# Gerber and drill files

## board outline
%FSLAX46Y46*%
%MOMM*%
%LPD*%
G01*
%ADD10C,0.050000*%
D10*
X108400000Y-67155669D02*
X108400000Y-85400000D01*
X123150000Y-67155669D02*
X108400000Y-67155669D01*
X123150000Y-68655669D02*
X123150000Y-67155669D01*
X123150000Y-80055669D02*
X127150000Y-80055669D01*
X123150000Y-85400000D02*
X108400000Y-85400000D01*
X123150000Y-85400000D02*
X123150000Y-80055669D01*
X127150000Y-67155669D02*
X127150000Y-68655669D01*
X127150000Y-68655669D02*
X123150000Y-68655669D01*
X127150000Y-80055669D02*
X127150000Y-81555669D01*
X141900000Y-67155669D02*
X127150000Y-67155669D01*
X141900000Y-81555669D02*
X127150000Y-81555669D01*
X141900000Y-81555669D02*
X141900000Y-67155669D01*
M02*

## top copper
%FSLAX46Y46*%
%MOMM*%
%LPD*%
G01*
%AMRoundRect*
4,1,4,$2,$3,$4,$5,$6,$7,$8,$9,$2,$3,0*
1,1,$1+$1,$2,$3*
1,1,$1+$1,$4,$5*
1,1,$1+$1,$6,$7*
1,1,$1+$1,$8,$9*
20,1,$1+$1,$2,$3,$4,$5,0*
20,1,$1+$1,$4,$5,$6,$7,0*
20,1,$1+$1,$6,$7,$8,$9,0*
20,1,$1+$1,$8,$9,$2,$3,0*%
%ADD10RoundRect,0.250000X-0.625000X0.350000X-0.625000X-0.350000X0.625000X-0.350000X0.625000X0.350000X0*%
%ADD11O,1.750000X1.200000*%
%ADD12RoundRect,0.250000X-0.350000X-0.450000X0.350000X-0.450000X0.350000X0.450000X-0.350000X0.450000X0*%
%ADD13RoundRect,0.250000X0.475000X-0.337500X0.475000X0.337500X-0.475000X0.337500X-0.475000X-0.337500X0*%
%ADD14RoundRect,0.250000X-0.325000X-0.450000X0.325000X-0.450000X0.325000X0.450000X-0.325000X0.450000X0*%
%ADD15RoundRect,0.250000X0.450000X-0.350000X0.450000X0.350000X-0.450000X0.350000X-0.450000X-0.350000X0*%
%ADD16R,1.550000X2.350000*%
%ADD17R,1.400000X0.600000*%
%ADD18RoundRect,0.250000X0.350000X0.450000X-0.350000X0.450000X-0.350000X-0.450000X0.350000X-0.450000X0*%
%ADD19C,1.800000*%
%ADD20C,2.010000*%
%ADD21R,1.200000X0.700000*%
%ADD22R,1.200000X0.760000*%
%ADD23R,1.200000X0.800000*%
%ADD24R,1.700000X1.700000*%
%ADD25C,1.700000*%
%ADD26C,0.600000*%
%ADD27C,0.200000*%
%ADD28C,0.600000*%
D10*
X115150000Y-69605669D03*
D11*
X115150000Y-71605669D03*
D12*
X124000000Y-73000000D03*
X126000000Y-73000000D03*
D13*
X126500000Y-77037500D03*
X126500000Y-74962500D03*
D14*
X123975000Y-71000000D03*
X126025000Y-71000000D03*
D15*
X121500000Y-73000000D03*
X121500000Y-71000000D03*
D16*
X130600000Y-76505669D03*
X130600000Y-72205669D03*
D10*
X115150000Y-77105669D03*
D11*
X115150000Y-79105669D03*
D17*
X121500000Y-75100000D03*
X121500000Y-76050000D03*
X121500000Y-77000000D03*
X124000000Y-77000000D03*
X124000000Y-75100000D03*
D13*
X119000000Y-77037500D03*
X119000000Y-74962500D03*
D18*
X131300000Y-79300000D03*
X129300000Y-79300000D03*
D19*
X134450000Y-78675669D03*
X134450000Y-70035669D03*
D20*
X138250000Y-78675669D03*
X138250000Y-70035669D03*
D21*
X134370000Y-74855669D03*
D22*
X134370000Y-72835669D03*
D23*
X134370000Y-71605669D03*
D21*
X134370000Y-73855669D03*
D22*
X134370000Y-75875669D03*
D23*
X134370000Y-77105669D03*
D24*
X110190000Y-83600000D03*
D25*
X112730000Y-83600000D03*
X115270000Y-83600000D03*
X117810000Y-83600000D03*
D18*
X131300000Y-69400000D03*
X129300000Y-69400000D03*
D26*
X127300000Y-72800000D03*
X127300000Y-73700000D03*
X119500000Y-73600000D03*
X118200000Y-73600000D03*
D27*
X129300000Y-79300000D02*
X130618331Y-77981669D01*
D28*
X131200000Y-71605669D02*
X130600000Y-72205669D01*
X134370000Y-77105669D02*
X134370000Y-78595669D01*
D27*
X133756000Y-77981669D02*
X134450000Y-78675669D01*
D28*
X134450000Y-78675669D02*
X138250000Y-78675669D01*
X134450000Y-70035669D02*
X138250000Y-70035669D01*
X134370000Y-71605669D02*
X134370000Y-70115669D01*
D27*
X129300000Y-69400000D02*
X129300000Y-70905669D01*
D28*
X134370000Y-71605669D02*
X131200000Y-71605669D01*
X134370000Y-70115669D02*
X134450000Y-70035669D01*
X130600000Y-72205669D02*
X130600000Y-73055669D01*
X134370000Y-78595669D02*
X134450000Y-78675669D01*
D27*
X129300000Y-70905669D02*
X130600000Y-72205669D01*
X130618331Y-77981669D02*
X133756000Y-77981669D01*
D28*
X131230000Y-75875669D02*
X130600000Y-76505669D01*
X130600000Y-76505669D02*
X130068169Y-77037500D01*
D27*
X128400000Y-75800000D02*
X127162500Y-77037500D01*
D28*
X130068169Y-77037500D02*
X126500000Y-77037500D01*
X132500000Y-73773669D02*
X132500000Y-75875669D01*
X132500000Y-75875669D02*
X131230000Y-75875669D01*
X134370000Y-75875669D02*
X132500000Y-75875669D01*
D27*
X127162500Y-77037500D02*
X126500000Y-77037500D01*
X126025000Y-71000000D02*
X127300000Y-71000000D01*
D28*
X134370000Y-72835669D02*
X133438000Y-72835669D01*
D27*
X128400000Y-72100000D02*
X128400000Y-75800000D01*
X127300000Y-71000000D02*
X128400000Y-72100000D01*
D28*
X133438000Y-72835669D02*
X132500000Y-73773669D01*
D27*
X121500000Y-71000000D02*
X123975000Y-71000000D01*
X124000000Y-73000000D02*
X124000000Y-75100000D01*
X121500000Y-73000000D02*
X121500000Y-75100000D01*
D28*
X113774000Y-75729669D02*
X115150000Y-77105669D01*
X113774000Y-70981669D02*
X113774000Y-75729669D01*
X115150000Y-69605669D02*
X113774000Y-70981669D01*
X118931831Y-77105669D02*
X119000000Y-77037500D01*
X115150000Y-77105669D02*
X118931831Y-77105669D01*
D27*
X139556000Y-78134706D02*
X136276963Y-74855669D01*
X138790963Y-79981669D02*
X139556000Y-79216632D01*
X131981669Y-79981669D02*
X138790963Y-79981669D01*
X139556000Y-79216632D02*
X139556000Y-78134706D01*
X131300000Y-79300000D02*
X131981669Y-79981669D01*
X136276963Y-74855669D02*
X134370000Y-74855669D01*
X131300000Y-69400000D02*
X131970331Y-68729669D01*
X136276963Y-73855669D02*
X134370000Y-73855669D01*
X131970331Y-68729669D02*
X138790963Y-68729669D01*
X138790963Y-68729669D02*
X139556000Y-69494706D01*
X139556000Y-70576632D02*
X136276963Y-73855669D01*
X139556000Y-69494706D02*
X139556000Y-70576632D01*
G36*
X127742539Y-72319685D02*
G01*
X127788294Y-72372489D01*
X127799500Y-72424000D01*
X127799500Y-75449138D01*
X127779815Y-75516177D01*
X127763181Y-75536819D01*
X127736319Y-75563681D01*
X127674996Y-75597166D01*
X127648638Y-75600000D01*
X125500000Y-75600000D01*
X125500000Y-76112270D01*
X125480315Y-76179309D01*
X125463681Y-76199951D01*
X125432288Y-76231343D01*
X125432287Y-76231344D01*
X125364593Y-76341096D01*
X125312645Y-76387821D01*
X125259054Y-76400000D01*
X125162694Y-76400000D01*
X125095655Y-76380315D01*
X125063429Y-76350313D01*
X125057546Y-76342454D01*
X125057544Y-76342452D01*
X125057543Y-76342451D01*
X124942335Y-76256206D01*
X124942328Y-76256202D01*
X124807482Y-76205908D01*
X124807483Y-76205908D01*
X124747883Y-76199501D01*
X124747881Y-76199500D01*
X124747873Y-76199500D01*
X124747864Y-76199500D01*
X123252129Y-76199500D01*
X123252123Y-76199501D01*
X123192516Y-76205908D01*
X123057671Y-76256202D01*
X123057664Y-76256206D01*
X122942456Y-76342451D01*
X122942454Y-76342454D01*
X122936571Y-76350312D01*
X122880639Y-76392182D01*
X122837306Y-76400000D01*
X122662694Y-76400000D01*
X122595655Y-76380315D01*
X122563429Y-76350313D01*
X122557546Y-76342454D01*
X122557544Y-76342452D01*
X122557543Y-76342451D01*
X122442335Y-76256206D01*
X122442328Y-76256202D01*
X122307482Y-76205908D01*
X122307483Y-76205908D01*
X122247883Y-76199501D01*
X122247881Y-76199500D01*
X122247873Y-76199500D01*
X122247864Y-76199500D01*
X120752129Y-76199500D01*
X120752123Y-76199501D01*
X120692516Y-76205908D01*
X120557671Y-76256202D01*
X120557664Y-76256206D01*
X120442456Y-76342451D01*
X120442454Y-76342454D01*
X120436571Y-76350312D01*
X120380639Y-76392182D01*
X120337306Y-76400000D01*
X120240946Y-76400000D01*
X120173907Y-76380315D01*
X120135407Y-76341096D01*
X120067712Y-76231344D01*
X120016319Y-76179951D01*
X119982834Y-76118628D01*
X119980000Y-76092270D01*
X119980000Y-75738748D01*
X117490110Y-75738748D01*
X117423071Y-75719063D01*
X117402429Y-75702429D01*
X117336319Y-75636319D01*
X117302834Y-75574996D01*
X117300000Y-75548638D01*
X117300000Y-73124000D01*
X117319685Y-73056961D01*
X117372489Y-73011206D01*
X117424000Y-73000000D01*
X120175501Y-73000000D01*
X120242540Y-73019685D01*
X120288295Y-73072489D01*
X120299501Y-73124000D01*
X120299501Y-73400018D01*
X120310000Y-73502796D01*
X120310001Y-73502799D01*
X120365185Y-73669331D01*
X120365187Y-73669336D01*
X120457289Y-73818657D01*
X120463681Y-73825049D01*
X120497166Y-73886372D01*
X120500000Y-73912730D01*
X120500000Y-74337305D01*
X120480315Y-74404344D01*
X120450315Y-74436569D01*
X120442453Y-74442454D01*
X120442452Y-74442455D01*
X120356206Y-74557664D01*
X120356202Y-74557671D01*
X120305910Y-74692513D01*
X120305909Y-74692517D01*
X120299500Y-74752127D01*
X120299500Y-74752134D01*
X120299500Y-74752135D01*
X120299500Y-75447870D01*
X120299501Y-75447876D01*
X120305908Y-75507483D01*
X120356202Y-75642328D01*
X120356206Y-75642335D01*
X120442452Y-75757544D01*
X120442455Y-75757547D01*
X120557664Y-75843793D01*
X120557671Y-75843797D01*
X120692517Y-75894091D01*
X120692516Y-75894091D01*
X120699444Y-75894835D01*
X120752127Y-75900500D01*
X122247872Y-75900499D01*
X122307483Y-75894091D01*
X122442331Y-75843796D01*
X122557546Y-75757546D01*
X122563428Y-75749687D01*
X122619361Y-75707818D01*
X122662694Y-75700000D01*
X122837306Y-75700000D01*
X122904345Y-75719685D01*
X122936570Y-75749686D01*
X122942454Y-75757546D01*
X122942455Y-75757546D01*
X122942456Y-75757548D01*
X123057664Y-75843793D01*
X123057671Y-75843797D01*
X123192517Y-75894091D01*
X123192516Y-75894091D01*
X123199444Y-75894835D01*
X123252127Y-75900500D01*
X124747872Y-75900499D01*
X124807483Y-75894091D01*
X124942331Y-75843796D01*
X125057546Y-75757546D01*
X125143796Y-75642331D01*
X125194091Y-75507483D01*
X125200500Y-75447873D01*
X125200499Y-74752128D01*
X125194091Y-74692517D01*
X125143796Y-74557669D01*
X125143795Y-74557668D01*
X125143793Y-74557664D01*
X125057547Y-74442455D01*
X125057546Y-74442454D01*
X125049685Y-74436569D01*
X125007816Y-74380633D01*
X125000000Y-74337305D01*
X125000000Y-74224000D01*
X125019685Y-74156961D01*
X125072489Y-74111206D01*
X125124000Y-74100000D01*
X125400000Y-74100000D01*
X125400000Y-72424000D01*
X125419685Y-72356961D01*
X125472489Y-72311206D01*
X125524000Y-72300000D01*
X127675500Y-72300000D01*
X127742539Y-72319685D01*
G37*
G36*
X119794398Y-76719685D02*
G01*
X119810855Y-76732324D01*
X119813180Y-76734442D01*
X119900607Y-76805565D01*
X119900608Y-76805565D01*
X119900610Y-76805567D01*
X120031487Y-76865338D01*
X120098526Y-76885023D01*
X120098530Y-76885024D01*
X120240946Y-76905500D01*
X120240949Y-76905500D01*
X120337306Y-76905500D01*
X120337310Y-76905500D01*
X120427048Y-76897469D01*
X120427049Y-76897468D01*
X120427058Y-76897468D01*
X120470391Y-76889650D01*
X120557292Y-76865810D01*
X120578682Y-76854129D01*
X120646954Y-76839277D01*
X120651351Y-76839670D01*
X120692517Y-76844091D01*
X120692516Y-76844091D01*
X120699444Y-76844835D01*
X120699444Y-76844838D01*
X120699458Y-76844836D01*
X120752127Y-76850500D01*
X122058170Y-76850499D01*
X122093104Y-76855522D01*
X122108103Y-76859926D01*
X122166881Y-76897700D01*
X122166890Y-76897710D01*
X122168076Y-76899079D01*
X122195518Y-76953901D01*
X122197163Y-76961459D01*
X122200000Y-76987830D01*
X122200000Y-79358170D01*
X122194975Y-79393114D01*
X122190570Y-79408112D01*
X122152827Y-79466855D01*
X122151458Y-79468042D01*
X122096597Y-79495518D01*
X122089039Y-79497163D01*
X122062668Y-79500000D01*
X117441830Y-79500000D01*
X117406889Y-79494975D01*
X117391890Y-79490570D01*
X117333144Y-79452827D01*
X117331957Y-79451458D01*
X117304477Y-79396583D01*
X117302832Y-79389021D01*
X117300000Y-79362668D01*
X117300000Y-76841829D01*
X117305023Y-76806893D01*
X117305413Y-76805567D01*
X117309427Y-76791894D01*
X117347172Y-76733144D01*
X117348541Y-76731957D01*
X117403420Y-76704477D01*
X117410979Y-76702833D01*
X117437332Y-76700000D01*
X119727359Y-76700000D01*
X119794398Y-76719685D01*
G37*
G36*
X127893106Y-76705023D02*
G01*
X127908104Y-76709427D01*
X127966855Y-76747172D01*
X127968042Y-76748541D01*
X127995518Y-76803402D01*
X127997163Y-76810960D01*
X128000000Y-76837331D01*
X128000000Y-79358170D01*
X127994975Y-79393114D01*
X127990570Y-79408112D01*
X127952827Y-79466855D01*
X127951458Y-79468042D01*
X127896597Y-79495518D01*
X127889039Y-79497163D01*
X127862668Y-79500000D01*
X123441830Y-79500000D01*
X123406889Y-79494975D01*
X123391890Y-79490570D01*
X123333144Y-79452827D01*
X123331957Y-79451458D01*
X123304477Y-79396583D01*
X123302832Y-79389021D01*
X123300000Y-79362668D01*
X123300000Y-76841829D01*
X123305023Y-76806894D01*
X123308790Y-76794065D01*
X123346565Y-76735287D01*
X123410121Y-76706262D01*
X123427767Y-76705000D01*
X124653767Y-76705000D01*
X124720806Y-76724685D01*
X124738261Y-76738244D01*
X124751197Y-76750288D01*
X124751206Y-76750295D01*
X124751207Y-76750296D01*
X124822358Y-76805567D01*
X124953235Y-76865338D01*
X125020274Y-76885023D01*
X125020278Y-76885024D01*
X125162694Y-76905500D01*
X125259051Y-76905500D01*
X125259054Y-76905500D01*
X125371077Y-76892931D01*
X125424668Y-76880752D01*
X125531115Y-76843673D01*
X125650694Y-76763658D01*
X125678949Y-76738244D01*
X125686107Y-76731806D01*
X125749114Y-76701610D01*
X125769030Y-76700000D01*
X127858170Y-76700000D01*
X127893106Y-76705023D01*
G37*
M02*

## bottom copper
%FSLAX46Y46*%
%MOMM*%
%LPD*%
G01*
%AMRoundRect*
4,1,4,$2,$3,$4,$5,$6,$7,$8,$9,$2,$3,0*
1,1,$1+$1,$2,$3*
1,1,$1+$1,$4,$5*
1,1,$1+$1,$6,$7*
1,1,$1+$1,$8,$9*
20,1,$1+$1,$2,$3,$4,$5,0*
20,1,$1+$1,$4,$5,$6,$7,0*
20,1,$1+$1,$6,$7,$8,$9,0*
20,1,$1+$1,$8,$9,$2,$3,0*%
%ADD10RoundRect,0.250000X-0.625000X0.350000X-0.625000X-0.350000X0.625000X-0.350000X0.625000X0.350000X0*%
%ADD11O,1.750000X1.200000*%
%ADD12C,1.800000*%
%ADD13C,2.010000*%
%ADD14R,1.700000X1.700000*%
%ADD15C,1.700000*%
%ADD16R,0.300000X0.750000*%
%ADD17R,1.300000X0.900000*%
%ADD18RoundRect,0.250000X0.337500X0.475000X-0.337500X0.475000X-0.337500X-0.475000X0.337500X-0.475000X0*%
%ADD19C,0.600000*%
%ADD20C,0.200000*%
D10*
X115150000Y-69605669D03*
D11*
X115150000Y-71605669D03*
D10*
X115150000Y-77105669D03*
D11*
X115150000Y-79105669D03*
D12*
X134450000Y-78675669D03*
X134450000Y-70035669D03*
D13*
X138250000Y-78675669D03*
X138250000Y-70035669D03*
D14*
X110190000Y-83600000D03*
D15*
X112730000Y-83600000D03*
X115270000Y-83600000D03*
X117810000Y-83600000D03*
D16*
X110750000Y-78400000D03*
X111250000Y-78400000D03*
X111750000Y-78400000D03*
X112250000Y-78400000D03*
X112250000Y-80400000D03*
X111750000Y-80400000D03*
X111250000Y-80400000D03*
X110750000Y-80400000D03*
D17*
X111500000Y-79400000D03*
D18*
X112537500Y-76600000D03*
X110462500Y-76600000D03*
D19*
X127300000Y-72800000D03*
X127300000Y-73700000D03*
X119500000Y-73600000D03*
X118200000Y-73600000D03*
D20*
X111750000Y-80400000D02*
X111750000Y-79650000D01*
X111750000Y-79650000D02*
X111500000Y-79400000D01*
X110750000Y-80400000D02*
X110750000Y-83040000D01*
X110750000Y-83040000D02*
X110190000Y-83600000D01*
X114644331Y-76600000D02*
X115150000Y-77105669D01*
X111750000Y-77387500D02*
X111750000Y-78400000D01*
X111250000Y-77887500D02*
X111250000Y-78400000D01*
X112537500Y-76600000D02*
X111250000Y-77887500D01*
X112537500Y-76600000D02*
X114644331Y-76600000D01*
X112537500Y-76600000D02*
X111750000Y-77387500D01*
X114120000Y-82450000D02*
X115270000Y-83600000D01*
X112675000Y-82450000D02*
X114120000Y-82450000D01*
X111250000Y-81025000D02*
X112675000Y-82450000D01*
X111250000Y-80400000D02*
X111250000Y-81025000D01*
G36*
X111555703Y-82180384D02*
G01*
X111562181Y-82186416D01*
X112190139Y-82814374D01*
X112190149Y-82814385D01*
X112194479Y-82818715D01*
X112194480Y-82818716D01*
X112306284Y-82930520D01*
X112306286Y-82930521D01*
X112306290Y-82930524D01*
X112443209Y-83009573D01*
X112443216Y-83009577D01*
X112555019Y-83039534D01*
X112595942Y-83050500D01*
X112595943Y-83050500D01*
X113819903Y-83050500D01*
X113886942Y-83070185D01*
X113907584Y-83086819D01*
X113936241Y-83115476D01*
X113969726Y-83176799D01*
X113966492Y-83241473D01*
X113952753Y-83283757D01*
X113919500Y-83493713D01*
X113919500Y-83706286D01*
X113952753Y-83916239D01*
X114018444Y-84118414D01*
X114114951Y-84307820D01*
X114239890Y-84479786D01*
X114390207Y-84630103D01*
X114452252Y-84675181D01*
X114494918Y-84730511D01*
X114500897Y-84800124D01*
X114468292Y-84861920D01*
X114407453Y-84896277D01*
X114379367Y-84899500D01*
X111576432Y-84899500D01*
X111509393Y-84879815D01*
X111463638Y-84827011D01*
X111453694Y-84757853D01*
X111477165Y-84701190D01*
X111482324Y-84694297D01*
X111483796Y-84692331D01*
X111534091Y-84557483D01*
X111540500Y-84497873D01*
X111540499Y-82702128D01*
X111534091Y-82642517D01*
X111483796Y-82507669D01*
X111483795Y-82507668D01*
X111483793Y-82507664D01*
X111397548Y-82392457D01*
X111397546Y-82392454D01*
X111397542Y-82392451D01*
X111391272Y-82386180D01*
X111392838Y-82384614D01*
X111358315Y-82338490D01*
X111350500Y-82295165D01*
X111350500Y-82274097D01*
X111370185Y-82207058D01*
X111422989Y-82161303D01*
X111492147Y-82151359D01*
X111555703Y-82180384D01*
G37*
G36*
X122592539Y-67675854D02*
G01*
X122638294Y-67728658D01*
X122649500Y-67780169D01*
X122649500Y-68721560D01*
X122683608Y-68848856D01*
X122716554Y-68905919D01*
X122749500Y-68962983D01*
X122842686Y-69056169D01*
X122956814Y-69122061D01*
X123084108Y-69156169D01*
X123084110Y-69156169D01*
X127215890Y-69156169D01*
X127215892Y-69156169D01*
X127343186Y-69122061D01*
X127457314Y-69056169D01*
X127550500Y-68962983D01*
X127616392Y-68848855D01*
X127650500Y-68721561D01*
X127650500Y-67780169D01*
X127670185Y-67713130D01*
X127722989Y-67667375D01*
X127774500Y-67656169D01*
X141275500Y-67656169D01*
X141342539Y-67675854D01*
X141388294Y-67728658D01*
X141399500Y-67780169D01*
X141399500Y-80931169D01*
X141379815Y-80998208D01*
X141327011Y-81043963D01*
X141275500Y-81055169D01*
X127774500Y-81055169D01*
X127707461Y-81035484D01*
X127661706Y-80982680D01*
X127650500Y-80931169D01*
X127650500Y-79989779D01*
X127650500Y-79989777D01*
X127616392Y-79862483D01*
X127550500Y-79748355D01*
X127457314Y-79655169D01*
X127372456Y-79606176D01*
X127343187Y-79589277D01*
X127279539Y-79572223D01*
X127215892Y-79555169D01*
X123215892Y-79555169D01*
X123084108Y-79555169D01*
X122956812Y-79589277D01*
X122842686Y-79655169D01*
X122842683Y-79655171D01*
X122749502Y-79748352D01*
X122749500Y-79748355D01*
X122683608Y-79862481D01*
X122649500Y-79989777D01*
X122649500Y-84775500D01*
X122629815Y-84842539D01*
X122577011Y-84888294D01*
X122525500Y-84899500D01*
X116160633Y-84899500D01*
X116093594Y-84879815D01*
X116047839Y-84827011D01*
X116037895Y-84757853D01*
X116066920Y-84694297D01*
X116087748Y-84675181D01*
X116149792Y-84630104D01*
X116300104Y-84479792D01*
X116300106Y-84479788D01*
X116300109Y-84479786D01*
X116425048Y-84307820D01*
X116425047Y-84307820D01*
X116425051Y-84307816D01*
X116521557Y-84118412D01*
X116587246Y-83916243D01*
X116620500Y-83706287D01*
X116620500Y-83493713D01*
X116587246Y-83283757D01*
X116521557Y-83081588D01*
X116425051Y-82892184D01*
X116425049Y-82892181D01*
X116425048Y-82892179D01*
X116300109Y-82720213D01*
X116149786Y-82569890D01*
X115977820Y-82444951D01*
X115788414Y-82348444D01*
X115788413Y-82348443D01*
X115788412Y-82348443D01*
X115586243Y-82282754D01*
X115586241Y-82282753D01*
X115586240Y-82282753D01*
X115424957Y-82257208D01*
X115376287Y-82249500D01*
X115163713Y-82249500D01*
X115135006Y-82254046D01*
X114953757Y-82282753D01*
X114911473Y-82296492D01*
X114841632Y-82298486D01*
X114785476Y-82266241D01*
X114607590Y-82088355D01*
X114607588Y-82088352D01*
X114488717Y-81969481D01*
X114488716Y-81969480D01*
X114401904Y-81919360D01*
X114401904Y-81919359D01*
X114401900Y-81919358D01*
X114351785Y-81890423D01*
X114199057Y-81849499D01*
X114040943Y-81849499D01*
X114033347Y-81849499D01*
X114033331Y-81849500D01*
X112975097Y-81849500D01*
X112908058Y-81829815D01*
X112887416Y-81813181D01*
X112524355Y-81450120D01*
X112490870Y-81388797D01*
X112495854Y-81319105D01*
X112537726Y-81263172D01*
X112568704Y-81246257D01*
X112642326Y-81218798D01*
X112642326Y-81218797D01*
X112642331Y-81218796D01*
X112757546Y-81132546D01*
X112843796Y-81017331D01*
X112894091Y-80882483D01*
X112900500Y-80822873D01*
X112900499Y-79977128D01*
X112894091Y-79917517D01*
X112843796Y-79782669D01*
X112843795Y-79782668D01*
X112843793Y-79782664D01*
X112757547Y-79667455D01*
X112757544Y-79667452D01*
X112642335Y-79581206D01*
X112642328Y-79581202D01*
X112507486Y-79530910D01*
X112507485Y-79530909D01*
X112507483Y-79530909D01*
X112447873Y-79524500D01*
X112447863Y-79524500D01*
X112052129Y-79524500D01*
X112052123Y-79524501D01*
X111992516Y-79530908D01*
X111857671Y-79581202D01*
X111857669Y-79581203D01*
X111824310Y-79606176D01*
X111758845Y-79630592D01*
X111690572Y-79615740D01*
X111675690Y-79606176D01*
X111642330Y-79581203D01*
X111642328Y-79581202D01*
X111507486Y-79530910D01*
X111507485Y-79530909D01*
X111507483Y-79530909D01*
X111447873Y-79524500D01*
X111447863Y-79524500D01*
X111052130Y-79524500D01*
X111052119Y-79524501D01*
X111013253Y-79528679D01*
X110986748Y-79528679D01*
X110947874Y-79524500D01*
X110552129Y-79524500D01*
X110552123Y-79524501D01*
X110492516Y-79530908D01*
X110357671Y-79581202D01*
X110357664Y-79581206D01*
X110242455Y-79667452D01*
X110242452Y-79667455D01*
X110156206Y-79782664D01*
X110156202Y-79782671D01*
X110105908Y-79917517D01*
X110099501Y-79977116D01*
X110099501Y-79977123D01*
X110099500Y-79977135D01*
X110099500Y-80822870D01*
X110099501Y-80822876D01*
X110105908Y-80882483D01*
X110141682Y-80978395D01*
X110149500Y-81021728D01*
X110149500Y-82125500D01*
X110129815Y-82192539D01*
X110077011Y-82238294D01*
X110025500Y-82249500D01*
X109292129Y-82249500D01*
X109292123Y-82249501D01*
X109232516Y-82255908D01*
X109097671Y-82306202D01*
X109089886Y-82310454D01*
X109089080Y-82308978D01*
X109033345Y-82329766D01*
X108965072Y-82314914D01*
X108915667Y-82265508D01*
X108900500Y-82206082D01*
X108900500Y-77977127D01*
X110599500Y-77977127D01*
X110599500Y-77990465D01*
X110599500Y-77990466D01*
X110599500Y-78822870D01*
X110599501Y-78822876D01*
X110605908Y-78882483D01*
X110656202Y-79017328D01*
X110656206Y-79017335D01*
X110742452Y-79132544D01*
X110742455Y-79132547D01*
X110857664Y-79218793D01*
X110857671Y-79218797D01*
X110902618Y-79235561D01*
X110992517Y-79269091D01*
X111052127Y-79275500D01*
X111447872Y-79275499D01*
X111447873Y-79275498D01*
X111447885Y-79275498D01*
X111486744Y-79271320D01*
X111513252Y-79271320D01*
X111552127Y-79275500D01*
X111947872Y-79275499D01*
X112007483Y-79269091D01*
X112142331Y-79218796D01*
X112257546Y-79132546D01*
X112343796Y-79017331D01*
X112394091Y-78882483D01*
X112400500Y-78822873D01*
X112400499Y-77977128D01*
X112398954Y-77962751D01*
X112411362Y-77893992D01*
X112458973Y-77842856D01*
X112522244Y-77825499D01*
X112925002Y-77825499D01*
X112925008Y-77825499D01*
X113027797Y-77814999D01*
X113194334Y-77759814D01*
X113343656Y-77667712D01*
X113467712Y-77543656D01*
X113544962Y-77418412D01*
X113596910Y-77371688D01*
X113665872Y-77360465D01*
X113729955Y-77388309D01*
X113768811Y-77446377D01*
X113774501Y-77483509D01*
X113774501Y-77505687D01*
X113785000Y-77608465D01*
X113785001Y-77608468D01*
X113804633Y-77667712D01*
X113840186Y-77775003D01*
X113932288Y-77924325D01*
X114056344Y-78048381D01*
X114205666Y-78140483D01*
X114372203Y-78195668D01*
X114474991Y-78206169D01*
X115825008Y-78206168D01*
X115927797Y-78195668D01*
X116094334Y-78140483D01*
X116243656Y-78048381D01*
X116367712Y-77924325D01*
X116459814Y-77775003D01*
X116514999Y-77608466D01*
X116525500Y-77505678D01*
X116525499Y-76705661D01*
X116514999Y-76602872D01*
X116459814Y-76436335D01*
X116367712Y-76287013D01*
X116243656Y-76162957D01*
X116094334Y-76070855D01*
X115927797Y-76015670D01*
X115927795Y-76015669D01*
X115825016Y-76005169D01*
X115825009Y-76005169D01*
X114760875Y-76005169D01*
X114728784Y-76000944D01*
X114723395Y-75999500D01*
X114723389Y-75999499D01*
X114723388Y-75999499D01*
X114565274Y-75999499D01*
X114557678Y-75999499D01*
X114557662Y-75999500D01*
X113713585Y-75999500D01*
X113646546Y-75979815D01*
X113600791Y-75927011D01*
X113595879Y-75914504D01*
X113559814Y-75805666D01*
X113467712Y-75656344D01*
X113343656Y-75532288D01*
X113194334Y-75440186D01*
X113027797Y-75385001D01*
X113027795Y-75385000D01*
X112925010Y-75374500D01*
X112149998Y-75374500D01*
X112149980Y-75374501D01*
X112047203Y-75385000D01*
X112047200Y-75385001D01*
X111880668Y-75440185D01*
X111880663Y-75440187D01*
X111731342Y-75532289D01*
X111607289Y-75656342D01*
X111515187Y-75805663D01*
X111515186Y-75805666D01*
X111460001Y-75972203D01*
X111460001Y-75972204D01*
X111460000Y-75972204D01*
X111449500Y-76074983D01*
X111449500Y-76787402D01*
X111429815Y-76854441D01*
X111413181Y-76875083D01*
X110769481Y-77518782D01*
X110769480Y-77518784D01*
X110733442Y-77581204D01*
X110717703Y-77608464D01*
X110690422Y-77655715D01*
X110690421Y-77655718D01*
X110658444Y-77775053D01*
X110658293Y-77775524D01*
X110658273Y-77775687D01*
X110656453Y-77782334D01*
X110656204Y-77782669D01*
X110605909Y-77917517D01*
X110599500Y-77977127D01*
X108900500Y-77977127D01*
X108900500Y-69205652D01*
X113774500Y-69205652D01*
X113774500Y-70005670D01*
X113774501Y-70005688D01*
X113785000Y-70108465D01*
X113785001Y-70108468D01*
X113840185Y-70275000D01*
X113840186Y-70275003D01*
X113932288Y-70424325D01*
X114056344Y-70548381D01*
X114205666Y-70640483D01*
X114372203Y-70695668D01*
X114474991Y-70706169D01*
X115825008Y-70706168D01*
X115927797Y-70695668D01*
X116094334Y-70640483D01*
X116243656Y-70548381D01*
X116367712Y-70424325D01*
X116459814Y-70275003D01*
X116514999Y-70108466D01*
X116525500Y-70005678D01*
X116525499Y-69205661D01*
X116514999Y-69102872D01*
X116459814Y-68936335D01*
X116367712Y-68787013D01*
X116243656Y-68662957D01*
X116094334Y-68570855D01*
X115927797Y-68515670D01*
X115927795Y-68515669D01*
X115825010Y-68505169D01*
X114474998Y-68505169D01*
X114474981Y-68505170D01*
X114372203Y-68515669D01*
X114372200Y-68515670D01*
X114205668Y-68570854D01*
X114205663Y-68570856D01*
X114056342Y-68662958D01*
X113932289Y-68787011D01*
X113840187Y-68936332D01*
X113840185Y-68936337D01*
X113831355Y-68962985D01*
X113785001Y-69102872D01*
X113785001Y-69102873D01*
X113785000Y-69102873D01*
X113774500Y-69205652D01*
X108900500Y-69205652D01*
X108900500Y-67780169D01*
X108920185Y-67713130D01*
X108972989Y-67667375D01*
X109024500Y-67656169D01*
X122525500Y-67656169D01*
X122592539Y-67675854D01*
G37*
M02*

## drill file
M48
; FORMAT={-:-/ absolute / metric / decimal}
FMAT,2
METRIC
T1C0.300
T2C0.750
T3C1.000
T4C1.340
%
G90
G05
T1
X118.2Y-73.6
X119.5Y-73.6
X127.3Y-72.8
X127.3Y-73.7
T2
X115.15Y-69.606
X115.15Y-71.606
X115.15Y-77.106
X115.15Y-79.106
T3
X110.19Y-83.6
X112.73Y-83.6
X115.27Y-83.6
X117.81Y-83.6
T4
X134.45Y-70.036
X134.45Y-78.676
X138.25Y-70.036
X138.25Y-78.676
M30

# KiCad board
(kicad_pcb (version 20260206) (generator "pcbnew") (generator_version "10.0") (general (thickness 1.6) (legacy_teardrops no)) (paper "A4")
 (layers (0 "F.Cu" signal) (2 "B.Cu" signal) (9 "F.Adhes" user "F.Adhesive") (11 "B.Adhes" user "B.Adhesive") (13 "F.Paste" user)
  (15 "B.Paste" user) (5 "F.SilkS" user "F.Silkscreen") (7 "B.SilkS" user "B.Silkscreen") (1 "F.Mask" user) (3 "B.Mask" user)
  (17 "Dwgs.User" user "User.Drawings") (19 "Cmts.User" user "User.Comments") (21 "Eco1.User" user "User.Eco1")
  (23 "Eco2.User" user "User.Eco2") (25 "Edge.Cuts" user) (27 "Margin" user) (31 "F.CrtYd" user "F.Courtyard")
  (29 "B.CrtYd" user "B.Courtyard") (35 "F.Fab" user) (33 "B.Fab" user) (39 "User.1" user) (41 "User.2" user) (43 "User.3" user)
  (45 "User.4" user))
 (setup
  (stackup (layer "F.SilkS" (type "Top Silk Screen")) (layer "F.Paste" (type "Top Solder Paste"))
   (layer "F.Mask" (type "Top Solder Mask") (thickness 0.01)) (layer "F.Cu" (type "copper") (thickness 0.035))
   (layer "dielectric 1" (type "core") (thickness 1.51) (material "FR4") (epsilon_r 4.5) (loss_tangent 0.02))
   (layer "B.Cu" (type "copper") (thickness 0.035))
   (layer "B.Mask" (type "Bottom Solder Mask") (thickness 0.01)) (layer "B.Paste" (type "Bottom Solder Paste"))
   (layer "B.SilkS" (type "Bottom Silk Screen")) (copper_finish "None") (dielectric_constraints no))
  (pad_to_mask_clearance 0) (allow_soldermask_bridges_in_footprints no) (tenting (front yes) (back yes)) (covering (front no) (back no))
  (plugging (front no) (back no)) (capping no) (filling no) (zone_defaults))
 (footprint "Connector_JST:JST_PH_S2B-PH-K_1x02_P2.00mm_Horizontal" (layer "F.Cu") (at 115.15 69.605669 -90)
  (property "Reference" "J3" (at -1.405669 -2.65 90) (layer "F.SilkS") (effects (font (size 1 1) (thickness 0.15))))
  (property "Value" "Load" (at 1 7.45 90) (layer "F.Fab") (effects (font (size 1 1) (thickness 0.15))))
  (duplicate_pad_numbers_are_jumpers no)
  (pad "1" thru_hole roundrect (at 0 0 270) (size 1.2 1.75) (drill 0.75) (layers "*.Cu" "*.Mask") (remove_unused_layers no)
   (roundrect_rratio 0.208333) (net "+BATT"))
  (pad "2" thru_hole oval (at 2 0 270) (size 1.2 1.75) (drill 0.75) (layers "*.Cu" "*.Mask") (remove_unused_layers no) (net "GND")))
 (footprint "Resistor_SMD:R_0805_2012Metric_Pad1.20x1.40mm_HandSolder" (layer "F.Cu") (at 125 73)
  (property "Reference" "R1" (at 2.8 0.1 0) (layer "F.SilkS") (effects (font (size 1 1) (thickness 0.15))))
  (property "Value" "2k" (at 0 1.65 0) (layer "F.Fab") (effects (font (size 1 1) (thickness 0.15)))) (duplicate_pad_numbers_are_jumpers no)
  (pad "1" smd roundrect (at -1 0) (size 1.2 1.4) (layers "F.Cu" "F.Mask" "F.Paste") (roundrect_rratio 0.208333) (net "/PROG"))
  (pad "2" smd roundrect (at 1 0) (size 1.2 1.4) (layers "F.Cu" "F.Mask" "F.Paste") (roundrect_rratio 0.208333) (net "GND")))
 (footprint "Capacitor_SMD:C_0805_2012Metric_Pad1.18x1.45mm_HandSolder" (layer "F.Cu") (at 126.5 76 90)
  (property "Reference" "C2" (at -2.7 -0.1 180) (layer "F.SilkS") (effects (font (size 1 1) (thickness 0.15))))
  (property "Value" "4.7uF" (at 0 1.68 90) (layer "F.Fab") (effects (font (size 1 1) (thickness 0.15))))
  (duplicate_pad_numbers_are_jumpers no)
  (pad "1" smd roundrect (at -1.0375 0 90) (size 1.175 1.45) (layers "F.Cu" "F.Mask" "F.Paste") (roundrect_rratio 0.212766) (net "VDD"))
  (pad "2" smd roundrect (at 1.0375 0 90) (size 1.175 1.45) (layers "F.Cu" "F.Mask" "F.Paste") (roundrect_rratio 0.212766) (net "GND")))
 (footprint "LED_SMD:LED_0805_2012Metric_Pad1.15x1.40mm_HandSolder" (layer "F.Cu") (at 125 71)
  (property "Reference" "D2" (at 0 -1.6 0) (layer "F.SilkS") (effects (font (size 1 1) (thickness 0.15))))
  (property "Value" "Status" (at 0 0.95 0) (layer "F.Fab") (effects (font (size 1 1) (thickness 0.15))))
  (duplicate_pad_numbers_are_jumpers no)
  (pad "1" smd roundrect (at -1.025 0) (size 1.15 1.4) (layers "F.Cu" "F.Mask" "F.Paste") (roundrect_rratio 0.217391) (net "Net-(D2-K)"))
  (pad "2" smd roundrect (at 1.025 0) (size 1.15 1.4) (layers "F.Cu" "F.Mask" "F.Paste") (roundrect_rratio 0.217391) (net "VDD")))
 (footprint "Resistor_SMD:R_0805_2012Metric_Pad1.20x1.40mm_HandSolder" (layer "F.Cu") (at 121.5 72 90)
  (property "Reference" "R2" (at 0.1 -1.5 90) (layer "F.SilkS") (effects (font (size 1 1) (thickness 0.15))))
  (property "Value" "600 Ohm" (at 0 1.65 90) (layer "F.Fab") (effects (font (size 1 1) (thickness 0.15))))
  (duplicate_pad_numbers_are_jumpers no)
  (pad "1" smd roundrect (at -1 0 90) (size 1.2 1.4) (layers "F.Cu" "F.Mask" "F.Paste") (roundrect_rratio 0.208333) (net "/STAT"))
  (pad "2" smd roundrect (at 1 0 90) (size 1.2 1.4) (layers "F.Cu" "F.Mask" "F.Paste") (roundrect_rratio 0.208333) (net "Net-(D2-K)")))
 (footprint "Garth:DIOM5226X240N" (layer "F.Cu") (at 130.6 74.355669 90)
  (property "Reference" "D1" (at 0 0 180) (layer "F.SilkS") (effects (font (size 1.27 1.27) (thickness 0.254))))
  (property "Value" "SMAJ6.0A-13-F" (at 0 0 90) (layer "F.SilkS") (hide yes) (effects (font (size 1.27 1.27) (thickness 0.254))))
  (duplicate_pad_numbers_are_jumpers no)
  (pad "1" smd rect (at -2.15 0 180) (size 1.55 2.35) (layers "F.Cu" "F.Mask" "F.Paste") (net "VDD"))
  (pad "2" smd rect (at 2.15 0 180) (size 1.55 2.35) (layers "F.Cu" "F.Mask" "F.Paste") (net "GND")))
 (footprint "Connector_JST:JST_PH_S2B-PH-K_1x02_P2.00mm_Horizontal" (layer "F.Cu") (at 115.15 77.105669 -90)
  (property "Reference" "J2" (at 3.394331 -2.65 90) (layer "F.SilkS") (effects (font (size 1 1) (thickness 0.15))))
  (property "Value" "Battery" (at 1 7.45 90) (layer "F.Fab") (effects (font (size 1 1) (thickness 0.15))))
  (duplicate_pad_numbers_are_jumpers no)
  (pad "1" thru_hole roundrect (at 0 0 270) (size 1.2 1.75) (drill 0.75) (layers "*.Cu" "*.Mask") (remove_unused_layers no)
   (roundrect_rratio 0.208333) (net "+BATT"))
  (pad "2" thru_hole oval (at 2 0 270) (size 1.2 1.75) (drill 0.75) (layers "*.Cu" "*.Mask") (remove_unused_layers no) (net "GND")))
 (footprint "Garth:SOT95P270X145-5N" (layer "F.Cu") (at 122.75 76.05)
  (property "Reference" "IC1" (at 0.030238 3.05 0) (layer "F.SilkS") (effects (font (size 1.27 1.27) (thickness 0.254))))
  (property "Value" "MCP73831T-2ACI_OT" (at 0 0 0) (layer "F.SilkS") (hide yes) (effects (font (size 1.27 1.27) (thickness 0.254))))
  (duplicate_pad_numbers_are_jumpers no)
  (pad "1" smd rect (at -1.25 -0.95 90) (size 0.6 1.4) (layers "F.Cu" "F.Mask" "F.Paste") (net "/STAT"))
  (pad "2" smd rect (at -1.25 0 90) (size 0.6 1.4) (layers "F.Cu" "F.Mask" "F.Paste") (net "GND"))
  (pad "3" smd rect (at -1.25 0.95 90) (size 0.6 1.4) (layers "F.Cu" "F.Mask" "F.Paste") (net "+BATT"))
  (pad "4" smd rect (at 1.25 0.95 90) (size 0.6 1.4) (layers "F.Cu" "F.Mask" "F.Paste") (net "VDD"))
  (pad "5" smd rect (at 1.25 -0.95 90) (size 0.6 1.4) (layers "F.Cu" "F.Mask" "F.Paste") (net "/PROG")))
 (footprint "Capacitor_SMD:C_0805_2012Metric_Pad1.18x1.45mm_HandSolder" (layer "F.Cu") (at 119 76 90)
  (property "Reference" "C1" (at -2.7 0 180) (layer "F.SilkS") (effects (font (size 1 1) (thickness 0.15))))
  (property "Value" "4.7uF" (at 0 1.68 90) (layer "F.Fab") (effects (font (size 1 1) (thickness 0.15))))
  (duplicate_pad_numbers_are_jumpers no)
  (pad "1" smd roundrect (at -1.0375 0 90) (size 1.175 1.45) (layers "F.Cu" "F.Mask" "F.Paste") (roundrect_rratio 0.212766) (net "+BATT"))
  (pad "2" smd roundrect (at 1.0375 0 90) (size 1.175 1.45) (layers "F.Cu" "F.Mask" "F.Paste") (roundrect_rratio 0.212766) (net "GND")))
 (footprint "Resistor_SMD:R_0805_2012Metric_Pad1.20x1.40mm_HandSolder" (layer "F.Cu") (at 130.3 79.3 180)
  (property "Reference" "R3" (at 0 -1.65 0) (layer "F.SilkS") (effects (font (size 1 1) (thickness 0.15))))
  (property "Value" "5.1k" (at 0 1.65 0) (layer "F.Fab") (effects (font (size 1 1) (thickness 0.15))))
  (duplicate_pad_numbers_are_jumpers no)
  (pad "1" smd roundrect (at -1 0 180) (size 1.2 1.4) (layers "F.Cu" "F.Mask" "F.Paste") (roundrect_rratio 0.208333) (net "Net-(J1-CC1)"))
  (pad "2" smd roundrect (at 1 0 180) (size 1.2 1.4) (layers "F.Cu" "F.Mask" "F.Paste") (roundrect_rratio 0.208333) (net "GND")))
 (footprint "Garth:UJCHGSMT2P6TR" (layer "F.Cu") (at 137.4 74.355669 90)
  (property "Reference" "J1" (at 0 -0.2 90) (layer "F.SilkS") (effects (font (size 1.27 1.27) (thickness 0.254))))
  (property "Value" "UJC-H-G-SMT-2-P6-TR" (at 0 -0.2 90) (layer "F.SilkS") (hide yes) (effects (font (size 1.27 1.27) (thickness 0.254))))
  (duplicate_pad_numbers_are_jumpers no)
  (pad "1" thru_hole circle (at -4.32 -2.95 90) (size 1.8 1.8) (drill 1.34) (layers "*.Cu" "*.Mask") (remove_unused_layers no) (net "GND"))
  (pad "2" thru_hole circle (at 4.32 -2.95 90) (size 1.8 1.8) (drill 1.34) (layers "*.Cu" "*.Mask") (remove_unused_layers no) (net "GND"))
  (pad "3" thru_hole circle (at -4.32 0.85 90) (size 2.01 2.01) (drill 1.34) (layers "*.Cu" "*.Mask") (remove_unused_layers no) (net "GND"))
  (pad "4" thru_hole circle (at 4.32 0.85 90) (size 2.01 2.01) (drill 1.34) (layers "*.Cu" "*.Mask") (remove_unused_layers no) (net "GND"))
  (pad "A5" smd rect (at -0.5 -3.03 90) (size 0.7 1.2) (layers "F.Cu" "F.Mask" "F.Paste") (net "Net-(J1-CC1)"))
  (pad "A9" smd rect (at 1.52 -3.03 90) (size 0.76 1.2) (layers "F.Cu" "F.Mask" "F.Paste") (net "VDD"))
  (pad "A12" smd rect (at 2.75 -3.03 90) (size 0.8 1.2) (layers "F.Cu" "F.Mask" "F.Paste") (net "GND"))
  (pad "B5" smd rect (at 0.5 -3.03 90) (size 0.7 1.2) (layers "F.Cu" "F.Mask" "F.Paste") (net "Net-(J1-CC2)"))
  (pad "B9" smd rect (at -1.52 -3.03 90) (size 0.76 1.2) (layers "F.Cu" "F.Mask" "F.Paste") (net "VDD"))
  (pad "B12" smd rect (at -2.75 -3.03 90) (size 0.8 1.2) (layers "F.Cu" "F.Mask" "F.Paste") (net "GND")))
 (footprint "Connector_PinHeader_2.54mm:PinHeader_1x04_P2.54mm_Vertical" (layer "F.Cu") (at 110.19 83.6 90)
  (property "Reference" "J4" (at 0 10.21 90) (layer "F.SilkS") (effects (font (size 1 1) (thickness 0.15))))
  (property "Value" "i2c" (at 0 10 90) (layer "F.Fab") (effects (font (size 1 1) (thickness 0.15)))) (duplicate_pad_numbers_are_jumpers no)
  (pad "1" thru_hole rect (at 0 0 90) (size 1.7 1.7) (drill 1) (layers "*.Cu" "*.Mask") (remove_unused_layers no) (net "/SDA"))
  (pad "2" thru_hole circle (at 0 2.54 90) (size 1.7 1.7) (drill 1) (layers "*.Cu" "*.Mask") (remove_unused_layers no) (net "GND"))
  (pad "3" thru_hole circle (at 0 5.08 90) (size 1.7 1.7) (drill 1) (layers "*.Cu" "*.Mask") (remove_unused_layers no) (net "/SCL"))
  (pad "4" thru_hole circle (at 0 7.62 90) (size 1.7 1.7) (drill 1) (layers "*.Cu" "*.Mask") (remove_unused_layers no) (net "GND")))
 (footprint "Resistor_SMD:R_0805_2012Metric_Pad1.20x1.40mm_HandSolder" (layer "F.Cu") (at 130.3 69.4 180)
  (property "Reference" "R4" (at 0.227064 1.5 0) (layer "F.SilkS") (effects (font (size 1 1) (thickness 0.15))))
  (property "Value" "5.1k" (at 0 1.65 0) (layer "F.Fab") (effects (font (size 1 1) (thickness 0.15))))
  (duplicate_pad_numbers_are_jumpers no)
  (pad "1" smd roundrect (at -1 0 180) (size 1.2 1.4) (layers "F.Cu" "F.Mask" "F.Paste") (roundrect_rratio 0.208333) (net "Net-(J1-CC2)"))
  (pad "2" smd roundrect (at 1 0 180) (size 1.2 1.4) (layers "F.Cu" "F.Mask" "F.Paste") (roundrect_rratio 0.208333) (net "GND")))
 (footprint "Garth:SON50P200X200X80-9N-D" (layer "B.Cu") (at 111.5 79.4 -90)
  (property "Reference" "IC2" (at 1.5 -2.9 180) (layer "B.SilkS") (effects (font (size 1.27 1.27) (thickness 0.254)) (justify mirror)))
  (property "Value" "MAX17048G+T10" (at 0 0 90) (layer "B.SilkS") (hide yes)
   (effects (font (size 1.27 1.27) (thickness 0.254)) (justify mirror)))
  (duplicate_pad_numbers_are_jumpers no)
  (pad "1" smd rect (at -1 0.75 180) (size 0.3 0.75) (layers "B.Cu" "B.Mask" "B.Paste") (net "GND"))
  (pad "2" smd rect (at -1 0.25 180) (size 0.3 0.75) (layers "B.Cu" "B.Mask" "B.Paste") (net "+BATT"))
  (pad "3" smd rect (at -1 -0.25 180) (size 0.3 0.75) (layers "B.Cu" "B.Mask" "B.Paste") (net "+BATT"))
  (pad "4" smd rect (at -1 -0.75 180) (size 0.3 0.75) (layers "B.Cu" "B.Mask" "B.Paste") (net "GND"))
  (pad "5" smd rect (at 1 -0.75 180) (size 0.3 0.75) (layers "B.Cu" "B.Mask" "B.Paste") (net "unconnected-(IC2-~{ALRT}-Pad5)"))
  (pad "6" smd rect (at 1 -0.25 180) (size 0.3 0.75) (layers "B.Cu" "B.Mask" "B.Paste") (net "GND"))
  (pad "7" smd rect (at 1 0.25 180) (size 0.3 0.75) (layers "B.Cu" "B.Mask" "B.Paste") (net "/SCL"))
  (pad "8" smd rect (at 1 0.75 180) (size 0.3 0.75) (layers "B.Cu" "B.Mask" "B.Paste") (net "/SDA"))
  (pad "9" smd rect (at 0 0 270) (size 0.9 1.3) (layers "B.Cu" "B.Mask" "B.Paste") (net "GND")))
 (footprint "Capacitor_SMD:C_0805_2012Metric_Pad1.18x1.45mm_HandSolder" (layer "B.Cu") (at 111.5 76.6 180)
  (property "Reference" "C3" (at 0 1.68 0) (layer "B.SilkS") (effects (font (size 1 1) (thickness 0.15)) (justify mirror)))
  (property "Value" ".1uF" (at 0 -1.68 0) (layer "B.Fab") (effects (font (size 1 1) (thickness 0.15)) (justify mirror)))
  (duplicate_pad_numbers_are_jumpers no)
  (pad "1" smd roundrect (at -1.0375 0 180) (size 1.175 1.45) (layers "B.Cu" "B.Mask" "B.Paste") (roundrect_rratio 0.212766) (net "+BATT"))
  (pad "2" smd roundrect (at 1.0375 0 180) (size 1.175 1.45) (layers "B.Cu" "B.Mask" "B.Paste") (roundrect_rratio 0.212766) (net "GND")))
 (gr_line (start 108.4 67.155669) (end 108.4 85.4) (stroke (width 0.05) (type default)) (layer "Edge.Cuts"))
 (gr_line (start 123.15 67.155669) (end 108.4 67.155669) (stroke (width 0.05) (type default)) (layer "Edge.Cuts"))
 (gr_line (start 123.15 68.655669) (end 123.15 67.155669) (stroke (width 0.05) (type default)) (layer "Edge.Cuts"))
 (gr_line (start 123.15 80.055669) (end 127.15 80.055669) (stroke (width 0.05) (type default)) (layer "Edge.Cuts"))
 (gr_line (start 123.15 85.4) (end 108.4 85.4) (stroke (width 0.05) (type default)) (layer "Edge.Cuts"))
 (gr_line (start 123.15 85.4) (end 123.15 80.055669) (stroke (width 0.05) (type default)) (layer "Edge.Cuts"))
 (gr_line (start 127.15 67.155669) (end 127.15 68.655669) (stroke (width 0.05) (type default)) (layer "Edge.Cuts"))
 (gr_line (start 127.15 68.655669) (end 123.15 68.655669) (stroke (width 0.05) (type default)) (layer "Edge.Cuts"))
 (gr_line (start 127.15 80.055669) (end 127.15 81.555669) (stroke (width 0.05) (type default)) (layer "Edge.Cuts"))
 (gr_line (start 141.9 67.155669) (end 127.15 67.155669) (stroke (width 0.05) (type default)) (layer "Edge.Cuts"))
 (gr_line (start 141.9 81.555669) (end 127.15 81.555669) (stroke (width 0.05) (type default)) (layer "Edge.Cuts"))
 (gr_line (start 141.9 81.555669) (end 141.9 67.155669) (stroke (width 0.05) (type default)) (layer "Edge.Cuts"))
 (segment (start 129.3 79.3) (end 130.618331 77.981669) (width 0.2) (layer "F.Cu") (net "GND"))
 (segment (start 131.2 71.605669) (end 130.6 72.205669) (width 0.6) (layer "F.Cu") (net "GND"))
 (segment (start 134.37 77.105669) (end 134.37 78.595669) (width 0.6) (layer "F.Cu") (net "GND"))
 (segment (start 133.756 77.981669) (end 134.45 78.675669) (width 0.2) (layer "F.Cu") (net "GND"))
 (segment (start 134.45 78.675669) (end 138.25 78.675669) (width 0.6) (layer "F.Cu") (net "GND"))
 (segment (start 134.45 70.035669) (end 138.25 70.035669) (width 0.6) (layer "F.Cu") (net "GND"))
 (segment (start 134.37 71.605669) (end 134.37 70.115669) (width 0.6) (layer "F.Cu") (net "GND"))
 (segment (start 129.3 69.4) (end 129.3 70.905669) (width 0.2) (layer "F.Cu") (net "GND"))
 (segment (start 134.37 71.605669) (end 131.2 71.605669) (width 0.6) (layer "F.Cu") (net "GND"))
 (segment (start 134.37 70.115669) (end 134.45 70.035669) (width 0.6) (layer "F.Cu") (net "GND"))
 (segment (start 130.6 72.205669) (end 130.6 73.055669) (width 0.6) (layer "F.Cu") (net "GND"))
 (segment (start 134.37 78.595669) (end 134.45 78.675669) (width 0.6) (layer "F.Cu") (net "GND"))
 (segment (start 129.3 70.905669) (end 130.6 72.205669) (width 0.2) (layer "F.Cu") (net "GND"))
 (segment (start 130.618331 77.981669) (end 133.756 77.981669) (width 0.2) (layer "F.Cu") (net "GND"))
 (via (at 127.3 72.8) (size 0.6) (drill 0.3) (layers "F.Cu" "B.Cu") (free yes) (capping no) (covering (front no) (back no))
  (plugging (front no) (back no)) (filling no) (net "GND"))
 (via (at 127.3 73.7) (size 0.6) (drill 0.3) (layers "F.Cu" "B.Cu") (free yes) (capping no) (covering (front no) (back no))
  (plugging (front no) (back no)) (filling no) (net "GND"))
 (via (at 119.5 73.6) (size 0.6) (drill 0.3) (layers "F.Cu" "B.Cu") (free yes) (capping no) (covering (front no) (back no))
  (plugging (front no) (back no)) (filling no) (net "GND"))
 (via (at 118.2 73.6) (size 0.6) (drill 0.3) (layers "F.Cu" "B.Cu") (free yes) (capping no) (covering (front no) (back no))
  (plugging (front no) (back no)) (filling no) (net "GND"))
 (segment (start 111.75 80.4) (end 111.75 79.65) (width 0.2) (layer "B.Cu") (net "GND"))
 (segment (start 111.75 79.65) (end 111.5 79.4) (width 0.2) (layer "B.Cu") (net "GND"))
 (segment (start 131.23 75.875669) (end 130.6 76.505669) (width 0.6) (layer "F.Cu") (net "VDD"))
 (segment (start 130.6 76.505669) (end 130.068169 77.0375) (width 0.6) (layer "F.Cu") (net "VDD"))
 (segment (start 128.4 75.8) (end 127.1625 77.0375) (width 0.2) (layer "F.Cu") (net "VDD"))
 (segment (start 130.068169 77.0375) (end 126.5 77.0375) (width 0.6) (layer "F.Cu") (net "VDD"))
 (segment (start 132.5 73.773669) (end 132.5 75.875669) (width 0.6) (layer "F.Cu") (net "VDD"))
 (segment (start 132.5 75.875669) (end 131.23 75.875669) (width 0.6) (layer "F.Cu") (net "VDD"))
 (segment (start 134.37 75.875669) (end 132.5 75.875669) (width 0.6) (layer "F.Cu") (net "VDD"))
 (segment (start 127.1625 77.0375) (end 126.5 77.0375) (width 0.2) (layer "F.Cu") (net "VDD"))
 (segment (start 126.025 71) (end 127.3 71) (width 0.2) (layer "F.Cu") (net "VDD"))
 (segment (start 134.37 72.835669) (end 133.438 72.835669) (width 0.6) (layer "F.Cu") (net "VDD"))
 (segment (start 128.4 72.1) (end 128.4 75.8) (width 0.2) (layer "F.Cu") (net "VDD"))
 (segment (start 127.3 71) (end 128.4 72.1) (width 0.2) (layer "F.Cu") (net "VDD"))
 (segment (start 133.438 72.835669) (end 132.5 73.773669) (width 0.6) (layer "F.Cu") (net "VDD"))
 (segment (start 121.5 71) (end 123.975 71) (width 0.2) (layer "F.Cu") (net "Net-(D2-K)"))
 (segment (start 110.75 80.4) (end 110.75 83.04) (width 0.2) (layer "B.Cu") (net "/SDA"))
 (segment (start 110.75 83.04) (end 110.19 83.6) (width 0.2) (layer "B.Cu") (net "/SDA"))
 (segment (start 124 73) (end 124 75.1) (width 0.2) (layer "F.Cu") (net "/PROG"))
 (segment (start 121.5 73) (end 121.5 75.1) (width 0.2) (layer "F.Cu") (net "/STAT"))
 (segment (start 113.774 75.729669) (end 115.15 77.105669) (width 0.6) (layer "F.Cu") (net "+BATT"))
 (segment (start 113.774 70.981669) (end 113.774 75.729669) (width 0.6) (layer "F.Cu") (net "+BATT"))
 (segment (start 115.15 69.605669) (end 113.774 70.981669) (width 0.6) (layer "F.Cu") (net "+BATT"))
 (segment (start 118.931831 77.105669) (end 119 77.0375) (width 0.6) (layer "F.Cu") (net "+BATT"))
 (segment (start 115.15 77.105669) (end 118.931831 77.105669) (width 0.6) (layer "F.Cu") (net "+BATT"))
 (segment (start 114.644331 76.6) (end 115.15 77.105669) (width 0.2) (layer "B.Cu") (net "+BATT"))
 (segment (start 111.75 77.3875) (end 111.75 78.4) (width 0.2) (layer "B.Cu") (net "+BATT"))
 (segment (start 111.25 77.8875) (end 111.25 78.4) (width 0.2) (layer "B.Cu") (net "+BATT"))
 (segment (start 112.5375 76.6) (end 111.25 77.8875) (width 0.2) (layer "B.Cu") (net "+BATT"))
 (segment (start 112.5375 76.6) (end 114.644331 76.6) (width 0.2) (layer "B.Cu") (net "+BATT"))
 (segment (start 112.5375 76.6) (end 111.75 77.3875) (width 0.2) (layer "B.Cu") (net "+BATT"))
 (segment (start 114.12 82.45) (end 115.27 83.6) (width 0.2) (layer "B.Cu") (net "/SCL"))
 (segment (start 112.675 82.45) (end 114.12 82.45) (width 0.2) (layer "B.Cu") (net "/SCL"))
 (segment (start 111.25 81.025) (end 112.675 82.45) (width 0.2) (layer "B.Cu") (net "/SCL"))
 (segment (start 111.25 80.4) (end 111.25 81.025) (width 0.2) (layer "B.Cu") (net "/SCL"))
 (segment (start 139.556 78.134706) (end 136.276963 74.855669) (width 0.2) (layer "F.Cu") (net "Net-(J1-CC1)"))
 (segment (start 138.790963 79.981669) (end 139.556 79.216632) (width 0.2) (layer "F.Cu") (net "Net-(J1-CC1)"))
 (segment (start 131.981669 79.981669) (end 138.790963 79.981669) (width 0.2) (layer "F.Cu") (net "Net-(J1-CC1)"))
 (segment (start 139.556 79.216632) (end 139.556 78.134706) (width 0.2) (layer "F.Cu") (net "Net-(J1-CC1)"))
 (segment (start 131.3 79.3) (end 131.981669 79.981669) (width 0.2) (layer "F.Cu") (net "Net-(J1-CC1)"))
 (segment (start 136.276963 74.855669) (end 134.37 74.855669) (width 0.2) (layer "F.Cu") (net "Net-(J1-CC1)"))
 (segment (start 131.3 69.4) (end 131.970331 68.729669) (width 0.2) (layer "F.Cu") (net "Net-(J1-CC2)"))
 (segment (start 136.276963 73.855669) (end 134.37 73.855669) (width 0.2) (layer "F.Cu") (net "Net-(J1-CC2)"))
 (segment (start 131.970331 68.729669) (end 138.790963 68.729669) (width 0.2) (layer "F.Cu") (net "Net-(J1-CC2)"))
 (segment (start 138.790963 68.729669) (end 139.556 69.494706) (width 0.2) (layer "F.Cu") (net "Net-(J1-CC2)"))
 (segment (start 139.556 70.576632) (end 136.276963 73.855669) (width 0.2) (layer "F.Cu") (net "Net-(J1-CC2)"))
 (segment (start 139.556 69.494706) (end 139.556 70.576632) (width 0.2) (layer "F.Cu") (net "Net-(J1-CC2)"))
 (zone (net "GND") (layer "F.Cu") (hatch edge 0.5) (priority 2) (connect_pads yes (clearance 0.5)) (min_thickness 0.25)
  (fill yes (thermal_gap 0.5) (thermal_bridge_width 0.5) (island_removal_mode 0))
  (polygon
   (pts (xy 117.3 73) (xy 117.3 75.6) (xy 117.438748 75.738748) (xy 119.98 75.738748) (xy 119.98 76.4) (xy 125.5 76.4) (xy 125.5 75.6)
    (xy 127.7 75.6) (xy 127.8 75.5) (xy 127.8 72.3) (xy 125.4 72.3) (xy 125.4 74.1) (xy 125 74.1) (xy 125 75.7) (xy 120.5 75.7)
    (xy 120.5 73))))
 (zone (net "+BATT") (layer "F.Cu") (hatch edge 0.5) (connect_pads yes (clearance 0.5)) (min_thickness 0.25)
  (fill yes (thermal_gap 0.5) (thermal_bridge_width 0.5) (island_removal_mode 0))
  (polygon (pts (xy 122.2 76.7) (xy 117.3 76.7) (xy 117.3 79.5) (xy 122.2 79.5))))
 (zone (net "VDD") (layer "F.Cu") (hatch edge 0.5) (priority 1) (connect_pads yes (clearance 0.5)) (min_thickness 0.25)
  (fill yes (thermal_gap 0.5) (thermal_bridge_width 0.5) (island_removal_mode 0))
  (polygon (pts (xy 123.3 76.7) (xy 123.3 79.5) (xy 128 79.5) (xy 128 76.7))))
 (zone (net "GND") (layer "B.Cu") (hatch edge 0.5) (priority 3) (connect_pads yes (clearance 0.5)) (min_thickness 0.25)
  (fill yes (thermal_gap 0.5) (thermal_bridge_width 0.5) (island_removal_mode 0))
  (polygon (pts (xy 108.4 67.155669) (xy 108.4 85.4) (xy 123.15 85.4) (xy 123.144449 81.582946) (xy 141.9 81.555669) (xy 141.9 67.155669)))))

